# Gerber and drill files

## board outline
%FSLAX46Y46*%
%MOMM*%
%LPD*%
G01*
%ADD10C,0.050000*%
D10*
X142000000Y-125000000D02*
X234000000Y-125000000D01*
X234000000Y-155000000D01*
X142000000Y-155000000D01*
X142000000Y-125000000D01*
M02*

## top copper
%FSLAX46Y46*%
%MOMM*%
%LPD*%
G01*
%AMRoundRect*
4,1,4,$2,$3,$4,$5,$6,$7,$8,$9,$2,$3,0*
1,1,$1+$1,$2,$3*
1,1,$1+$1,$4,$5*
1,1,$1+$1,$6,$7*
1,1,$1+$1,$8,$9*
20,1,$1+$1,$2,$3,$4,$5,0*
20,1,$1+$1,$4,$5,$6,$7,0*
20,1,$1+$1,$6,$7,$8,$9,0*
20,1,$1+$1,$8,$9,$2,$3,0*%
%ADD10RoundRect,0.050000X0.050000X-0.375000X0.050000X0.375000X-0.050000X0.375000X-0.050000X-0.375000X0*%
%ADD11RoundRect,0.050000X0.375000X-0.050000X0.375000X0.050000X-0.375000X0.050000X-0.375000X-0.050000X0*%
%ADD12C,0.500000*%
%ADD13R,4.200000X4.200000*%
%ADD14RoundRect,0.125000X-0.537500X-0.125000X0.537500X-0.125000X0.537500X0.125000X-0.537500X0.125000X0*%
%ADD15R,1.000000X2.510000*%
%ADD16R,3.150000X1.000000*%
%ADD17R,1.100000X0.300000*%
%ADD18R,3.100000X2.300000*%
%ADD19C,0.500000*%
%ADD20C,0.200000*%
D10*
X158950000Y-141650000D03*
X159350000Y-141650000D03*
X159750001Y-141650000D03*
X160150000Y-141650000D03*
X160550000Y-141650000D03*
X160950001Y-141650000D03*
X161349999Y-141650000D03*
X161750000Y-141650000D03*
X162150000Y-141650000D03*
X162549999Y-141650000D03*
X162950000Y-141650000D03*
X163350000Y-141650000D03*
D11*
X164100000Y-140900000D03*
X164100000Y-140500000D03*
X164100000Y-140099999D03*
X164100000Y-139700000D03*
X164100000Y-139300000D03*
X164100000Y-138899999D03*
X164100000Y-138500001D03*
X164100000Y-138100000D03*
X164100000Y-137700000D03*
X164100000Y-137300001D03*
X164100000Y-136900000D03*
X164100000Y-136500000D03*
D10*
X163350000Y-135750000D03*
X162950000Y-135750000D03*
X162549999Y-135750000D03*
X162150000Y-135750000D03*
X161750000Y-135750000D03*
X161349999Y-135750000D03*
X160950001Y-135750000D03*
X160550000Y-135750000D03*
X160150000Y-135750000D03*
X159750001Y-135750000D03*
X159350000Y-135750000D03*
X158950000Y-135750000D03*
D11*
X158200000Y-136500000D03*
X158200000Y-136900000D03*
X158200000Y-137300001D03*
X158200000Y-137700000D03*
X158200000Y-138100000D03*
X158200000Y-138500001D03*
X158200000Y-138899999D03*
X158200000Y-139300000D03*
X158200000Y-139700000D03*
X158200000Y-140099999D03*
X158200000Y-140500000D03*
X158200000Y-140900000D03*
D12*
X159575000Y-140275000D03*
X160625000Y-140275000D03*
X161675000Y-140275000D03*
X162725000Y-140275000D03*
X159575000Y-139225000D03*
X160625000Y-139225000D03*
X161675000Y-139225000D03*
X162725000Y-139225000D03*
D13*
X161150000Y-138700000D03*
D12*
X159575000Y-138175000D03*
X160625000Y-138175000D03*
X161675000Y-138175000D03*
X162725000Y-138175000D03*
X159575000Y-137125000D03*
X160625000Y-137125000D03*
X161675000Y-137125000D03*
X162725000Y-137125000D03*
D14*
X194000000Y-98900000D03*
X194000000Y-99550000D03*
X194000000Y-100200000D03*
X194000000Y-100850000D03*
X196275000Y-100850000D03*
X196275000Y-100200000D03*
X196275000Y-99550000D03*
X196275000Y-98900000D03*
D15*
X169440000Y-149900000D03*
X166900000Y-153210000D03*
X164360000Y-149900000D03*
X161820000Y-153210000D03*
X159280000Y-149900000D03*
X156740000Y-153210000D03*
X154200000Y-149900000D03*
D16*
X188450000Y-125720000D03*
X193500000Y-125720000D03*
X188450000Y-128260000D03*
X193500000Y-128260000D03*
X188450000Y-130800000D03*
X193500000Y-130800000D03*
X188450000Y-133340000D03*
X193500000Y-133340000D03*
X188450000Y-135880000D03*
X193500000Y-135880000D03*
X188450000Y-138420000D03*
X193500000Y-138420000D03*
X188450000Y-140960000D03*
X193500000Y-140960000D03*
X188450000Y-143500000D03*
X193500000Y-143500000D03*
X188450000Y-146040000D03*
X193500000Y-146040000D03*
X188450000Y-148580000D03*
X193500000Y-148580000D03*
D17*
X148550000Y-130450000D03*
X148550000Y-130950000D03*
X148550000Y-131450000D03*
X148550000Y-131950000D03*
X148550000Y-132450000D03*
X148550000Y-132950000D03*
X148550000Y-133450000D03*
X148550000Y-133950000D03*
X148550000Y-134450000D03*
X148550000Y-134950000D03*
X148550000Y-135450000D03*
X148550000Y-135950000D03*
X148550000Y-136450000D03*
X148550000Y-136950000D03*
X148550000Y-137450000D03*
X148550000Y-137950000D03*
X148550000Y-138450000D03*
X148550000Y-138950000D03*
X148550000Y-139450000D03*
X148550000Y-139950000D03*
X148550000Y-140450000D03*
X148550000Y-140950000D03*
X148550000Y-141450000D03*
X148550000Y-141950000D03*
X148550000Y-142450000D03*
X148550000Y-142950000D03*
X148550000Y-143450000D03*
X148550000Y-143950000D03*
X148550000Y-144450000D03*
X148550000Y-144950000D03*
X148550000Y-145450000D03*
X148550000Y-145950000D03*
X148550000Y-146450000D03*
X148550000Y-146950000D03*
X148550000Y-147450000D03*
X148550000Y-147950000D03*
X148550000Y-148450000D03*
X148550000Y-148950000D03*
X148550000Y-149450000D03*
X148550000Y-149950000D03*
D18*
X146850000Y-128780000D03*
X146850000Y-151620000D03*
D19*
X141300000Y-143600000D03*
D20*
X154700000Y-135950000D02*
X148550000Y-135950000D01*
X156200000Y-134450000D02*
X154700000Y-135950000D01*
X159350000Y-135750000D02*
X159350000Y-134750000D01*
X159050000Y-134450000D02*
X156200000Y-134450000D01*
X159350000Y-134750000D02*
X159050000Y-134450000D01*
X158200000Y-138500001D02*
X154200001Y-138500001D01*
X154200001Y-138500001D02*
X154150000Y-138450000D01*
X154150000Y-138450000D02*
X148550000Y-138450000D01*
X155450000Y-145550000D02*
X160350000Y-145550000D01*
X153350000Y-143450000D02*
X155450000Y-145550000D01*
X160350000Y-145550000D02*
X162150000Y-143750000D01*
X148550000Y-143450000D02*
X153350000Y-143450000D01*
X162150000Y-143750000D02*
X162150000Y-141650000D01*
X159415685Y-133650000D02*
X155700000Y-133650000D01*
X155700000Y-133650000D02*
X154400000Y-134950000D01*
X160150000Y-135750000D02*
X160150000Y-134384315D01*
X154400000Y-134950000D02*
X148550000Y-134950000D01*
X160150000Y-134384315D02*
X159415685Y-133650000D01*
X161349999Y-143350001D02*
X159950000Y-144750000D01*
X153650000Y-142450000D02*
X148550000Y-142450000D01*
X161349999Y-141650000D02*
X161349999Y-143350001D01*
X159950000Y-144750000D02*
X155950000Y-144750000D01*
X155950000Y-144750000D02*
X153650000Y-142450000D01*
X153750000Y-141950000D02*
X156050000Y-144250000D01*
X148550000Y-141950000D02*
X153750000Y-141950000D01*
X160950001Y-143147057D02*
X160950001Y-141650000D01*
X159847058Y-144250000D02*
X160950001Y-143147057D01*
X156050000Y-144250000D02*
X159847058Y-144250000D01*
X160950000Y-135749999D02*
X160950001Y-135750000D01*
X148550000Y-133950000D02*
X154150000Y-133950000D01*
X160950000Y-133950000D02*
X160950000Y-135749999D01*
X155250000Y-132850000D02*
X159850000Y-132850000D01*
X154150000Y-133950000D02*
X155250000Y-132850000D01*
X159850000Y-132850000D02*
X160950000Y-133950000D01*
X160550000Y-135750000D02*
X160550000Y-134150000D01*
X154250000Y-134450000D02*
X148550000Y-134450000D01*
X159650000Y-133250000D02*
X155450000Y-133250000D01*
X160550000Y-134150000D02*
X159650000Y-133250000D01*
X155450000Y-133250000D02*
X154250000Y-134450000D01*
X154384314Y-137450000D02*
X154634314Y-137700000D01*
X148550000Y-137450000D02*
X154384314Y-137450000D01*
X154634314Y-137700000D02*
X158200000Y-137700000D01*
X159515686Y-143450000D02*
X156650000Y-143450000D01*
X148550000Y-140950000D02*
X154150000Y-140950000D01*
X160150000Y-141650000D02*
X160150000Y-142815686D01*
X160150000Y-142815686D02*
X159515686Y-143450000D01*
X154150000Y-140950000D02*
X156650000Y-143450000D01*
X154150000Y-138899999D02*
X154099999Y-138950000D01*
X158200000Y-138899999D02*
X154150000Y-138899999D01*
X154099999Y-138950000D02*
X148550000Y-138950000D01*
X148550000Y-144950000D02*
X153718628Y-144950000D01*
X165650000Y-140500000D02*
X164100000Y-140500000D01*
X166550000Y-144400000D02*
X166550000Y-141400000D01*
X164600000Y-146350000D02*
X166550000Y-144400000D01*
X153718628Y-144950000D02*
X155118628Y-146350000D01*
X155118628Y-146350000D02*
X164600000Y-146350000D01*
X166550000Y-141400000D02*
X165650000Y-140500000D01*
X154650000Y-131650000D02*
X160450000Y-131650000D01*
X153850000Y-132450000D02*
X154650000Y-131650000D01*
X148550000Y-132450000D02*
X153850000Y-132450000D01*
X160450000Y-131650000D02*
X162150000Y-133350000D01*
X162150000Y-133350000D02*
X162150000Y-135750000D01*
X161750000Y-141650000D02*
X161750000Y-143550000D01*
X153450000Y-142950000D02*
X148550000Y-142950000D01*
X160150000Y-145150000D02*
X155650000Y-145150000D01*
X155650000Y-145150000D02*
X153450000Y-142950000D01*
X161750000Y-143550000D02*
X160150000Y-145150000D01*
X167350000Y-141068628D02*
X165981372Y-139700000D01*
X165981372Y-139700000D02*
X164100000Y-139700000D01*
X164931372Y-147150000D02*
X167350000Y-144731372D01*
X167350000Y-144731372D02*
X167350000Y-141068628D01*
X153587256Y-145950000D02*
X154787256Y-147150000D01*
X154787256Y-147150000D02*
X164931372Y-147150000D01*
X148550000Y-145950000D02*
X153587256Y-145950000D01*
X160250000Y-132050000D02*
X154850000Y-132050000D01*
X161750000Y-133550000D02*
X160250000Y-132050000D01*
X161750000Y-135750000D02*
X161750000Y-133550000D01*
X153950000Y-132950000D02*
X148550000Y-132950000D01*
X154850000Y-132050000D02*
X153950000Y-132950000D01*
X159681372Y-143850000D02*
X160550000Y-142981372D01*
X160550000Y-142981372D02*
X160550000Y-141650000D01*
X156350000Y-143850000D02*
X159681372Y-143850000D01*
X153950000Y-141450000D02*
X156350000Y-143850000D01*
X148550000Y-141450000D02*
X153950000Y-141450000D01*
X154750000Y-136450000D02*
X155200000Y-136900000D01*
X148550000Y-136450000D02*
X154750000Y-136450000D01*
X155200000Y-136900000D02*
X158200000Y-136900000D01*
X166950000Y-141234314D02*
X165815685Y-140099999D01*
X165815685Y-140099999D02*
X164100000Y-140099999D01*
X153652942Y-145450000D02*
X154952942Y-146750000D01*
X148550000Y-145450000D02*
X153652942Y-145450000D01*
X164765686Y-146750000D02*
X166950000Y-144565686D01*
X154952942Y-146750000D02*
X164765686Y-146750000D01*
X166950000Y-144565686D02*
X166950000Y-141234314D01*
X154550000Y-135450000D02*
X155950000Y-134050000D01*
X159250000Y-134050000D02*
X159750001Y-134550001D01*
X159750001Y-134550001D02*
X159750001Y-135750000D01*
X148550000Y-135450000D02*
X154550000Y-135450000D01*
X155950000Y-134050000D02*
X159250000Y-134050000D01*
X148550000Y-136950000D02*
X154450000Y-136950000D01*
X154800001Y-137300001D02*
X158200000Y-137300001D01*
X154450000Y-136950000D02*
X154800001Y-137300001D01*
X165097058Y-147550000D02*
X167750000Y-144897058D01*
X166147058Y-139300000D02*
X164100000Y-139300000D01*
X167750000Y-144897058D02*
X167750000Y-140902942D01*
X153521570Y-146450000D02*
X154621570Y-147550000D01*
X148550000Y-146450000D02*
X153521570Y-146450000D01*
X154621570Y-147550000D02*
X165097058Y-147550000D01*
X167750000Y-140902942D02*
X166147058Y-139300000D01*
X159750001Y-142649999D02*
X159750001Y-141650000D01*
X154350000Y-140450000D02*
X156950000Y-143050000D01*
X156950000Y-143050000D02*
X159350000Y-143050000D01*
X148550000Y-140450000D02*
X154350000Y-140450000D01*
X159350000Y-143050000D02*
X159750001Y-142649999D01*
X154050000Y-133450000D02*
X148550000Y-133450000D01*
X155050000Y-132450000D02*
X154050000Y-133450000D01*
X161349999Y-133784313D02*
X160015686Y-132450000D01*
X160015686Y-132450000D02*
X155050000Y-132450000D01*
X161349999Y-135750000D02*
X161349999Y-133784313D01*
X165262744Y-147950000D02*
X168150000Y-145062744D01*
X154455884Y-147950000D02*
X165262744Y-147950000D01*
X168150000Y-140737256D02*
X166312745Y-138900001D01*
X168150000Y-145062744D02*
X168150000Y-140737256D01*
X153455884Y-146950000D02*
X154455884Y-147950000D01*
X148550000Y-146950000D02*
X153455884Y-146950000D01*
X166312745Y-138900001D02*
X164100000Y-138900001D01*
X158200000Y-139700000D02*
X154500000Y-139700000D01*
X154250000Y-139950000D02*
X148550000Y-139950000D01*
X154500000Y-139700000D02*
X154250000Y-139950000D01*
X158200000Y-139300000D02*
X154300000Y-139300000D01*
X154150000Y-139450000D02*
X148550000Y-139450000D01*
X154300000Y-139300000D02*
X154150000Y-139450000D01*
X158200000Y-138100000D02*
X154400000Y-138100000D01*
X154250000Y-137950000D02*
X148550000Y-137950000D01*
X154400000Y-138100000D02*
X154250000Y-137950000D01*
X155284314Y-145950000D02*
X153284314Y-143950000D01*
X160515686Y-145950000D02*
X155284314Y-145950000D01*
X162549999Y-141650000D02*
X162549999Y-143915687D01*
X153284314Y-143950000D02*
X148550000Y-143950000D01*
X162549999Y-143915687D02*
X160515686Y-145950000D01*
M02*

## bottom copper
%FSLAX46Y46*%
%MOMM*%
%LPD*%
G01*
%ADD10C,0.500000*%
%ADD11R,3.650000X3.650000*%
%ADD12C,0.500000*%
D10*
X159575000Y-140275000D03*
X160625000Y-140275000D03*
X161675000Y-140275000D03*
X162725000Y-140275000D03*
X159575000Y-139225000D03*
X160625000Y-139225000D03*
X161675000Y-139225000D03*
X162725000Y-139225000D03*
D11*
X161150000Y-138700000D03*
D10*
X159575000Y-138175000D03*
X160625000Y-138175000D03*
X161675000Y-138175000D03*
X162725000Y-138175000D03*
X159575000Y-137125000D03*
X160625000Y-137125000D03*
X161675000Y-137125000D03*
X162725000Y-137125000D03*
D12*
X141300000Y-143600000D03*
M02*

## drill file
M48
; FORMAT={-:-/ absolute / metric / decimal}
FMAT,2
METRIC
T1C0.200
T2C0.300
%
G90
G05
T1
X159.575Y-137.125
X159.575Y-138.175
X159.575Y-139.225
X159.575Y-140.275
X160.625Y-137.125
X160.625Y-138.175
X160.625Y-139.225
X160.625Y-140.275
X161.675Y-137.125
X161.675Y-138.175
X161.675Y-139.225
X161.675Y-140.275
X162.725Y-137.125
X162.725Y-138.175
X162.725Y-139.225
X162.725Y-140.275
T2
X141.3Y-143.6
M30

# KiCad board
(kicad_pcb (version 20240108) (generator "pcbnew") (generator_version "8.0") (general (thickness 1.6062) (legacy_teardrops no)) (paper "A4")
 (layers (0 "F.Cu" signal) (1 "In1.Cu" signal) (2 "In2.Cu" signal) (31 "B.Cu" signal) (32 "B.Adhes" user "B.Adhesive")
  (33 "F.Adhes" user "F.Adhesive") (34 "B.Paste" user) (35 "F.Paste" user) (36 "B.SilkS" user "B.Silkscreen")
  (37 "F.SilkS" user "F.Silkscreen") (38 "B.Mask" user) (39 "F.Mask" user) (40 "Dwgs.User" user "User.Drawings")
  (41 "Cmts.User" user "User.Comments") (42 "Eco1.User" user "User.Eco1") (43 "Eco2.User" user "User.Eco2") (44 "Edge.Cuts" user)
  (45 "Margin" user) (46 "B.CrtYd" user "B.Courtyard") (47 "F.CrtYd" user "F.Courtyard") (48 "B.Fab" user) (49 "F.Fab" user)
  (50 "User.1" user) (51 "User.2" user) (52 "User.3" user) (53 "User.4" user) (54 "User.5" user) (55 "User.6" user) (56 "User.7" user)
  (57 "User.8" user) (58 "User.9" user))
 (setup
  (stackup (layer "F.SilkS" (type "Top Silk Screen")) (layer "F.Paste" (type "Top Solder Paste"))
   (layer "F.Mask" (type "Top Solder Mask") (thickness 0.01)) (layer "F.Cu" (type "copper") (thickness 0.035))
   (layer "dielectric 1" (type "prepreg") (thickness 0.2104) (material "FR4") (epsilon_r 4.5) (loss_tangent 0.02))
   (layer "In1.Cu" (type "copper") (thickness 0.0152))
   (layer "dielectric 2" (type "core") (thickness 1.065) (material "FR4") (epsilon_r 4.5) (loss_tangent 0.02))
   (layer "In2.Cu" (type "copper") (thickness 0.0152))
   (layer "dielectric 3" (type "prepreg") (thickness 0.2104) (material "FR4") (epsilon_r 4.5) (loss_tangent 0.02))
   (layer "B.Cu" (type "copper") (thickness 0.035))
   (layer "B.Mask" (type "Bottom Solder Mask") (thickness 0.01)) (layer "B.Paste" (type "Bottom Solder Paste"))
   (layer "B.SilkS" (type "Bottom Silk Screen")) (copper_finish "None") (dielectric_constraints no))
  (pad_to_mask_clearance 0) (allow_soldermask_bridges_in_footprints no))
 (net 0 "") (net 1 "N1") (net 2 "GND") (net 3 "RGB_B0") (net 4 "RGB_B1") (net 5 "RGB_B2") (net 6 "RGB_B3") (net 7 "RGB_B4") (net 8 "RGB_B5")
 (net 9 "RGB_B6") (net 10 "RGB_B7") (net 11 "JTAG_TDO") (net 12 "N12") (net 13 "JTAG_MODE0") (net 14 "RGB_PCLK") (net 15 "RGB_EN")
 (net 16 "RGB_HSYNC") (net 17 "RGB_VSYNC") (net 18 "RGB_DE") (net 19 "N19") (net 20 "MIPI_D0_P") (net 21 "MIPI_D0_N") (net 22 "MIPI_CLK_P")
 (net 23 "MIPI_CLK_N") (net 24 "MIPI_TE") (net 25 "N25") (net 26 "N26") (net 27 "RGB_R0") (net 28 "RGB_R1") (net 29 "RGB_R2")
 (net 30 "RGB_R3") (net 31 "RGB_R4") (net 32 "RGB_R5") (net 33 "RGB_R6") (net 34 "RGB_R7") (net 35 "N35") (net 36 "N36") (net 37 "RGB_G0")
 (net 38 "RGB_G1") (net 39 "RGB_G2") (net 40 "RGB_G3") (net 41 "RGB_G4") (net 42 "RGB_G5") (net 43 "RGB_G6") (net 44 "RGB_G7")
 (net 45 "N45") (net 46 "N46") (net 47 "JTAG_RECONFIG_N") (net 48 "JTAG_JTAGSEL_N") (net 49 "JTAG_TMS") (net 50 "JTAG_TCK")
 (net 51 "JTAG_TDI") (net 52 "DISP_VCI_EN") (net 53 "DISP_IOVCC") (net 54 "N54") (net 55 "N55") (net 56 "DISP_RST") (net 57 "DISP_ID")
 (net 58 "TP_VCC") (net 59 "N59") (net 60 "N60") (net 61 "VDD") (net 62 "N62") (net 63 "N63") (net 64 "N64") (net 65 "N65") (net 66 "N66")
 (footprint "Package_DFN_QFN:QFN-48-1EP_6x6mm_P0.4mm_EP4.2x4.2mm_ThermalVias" (layer "F.Cu") (at 161.15 138.7 90)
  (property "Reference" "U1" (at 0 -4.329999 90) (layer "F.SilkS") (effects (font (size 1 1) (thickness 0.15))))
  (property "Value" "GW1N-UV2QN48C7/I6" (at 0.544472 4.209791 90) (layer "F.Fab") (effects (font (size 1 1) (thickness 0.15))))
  (pad "" smd custom (at -1.8375 -1.8375 90) (size 0.295204 0.295204) (layers "F.Paste") (options (clearance outline) (anchor circle))
   (primitives))
  (pad "" smd custom (at -1.8375 -1.05 90) (size 0.331171 0.331171) (layers "F.Paste") (options (clearance outline) (anchor circle))
   (primitives))
  (pad "" smd custom (at -1.8375 0 90) (size 0.331171 0.331171) (layers "F.Paste") (options (clearance outline) (anchor circle))
   (primitives))
  (pad "" smd custom (at -1.8375 1.05 90) (size 0.331171 0.331171) (layers "F.Paste") (options (clearance outline) (anchor circle))
   (primitives))
  (pad "" smd custom (at -1.8375 1.8375 90) (size 0.295204 0.295204) (layers "F.Paste") (options (clearance outline) (anchor circle))
   (primitives))
  (pad "" smd custom (at -1.05 -1.8375 90) (size 0.331171 0.331171) (layers "F.Paste") (options (clearance outline) (anchor circle))
   (primitives))
  (pad "" smd roundrect (at -1.05 -1.05 90) (size 0.846537 0.846537) (layers "F.Paste") (roundrect_rratio 0.25))
  (pad "" smd roundrect (at -1.05 0 90) (size 0.846537 0.846537) (layers "F.Paste") (roundrect_rratio 0.25))
  (pad "" smd roundrect (at -1.05 1.05 90) (size 0.846537 0.846537) (layers "F.Paste") (roundrect_rratio 0.25))
  (pad "" smd custom (at -1.05 1.8375 90) (size 0.331171 0.331171) (layers "F.Paste") (options (clearance outline) (anchor circle))
   (primitives))
  (pad "" smd custom (at 0 -1.8375 90) (size 0.331171 0.331171) (layers "F.Paste") (options (clearance outline) (anchor circle))
   (primitives))
  (pad "" smd roundrect (at 0 -1.05 90) (size 0.846537 0.846537) (layers "F.Paste") (roundrect_rratio 0.25))
  (pad "" smd roundrect (at 0 0 90) (size 0.846537 0.846537) (layers "F.Paste") (roundrect_rratio 0.25))
  (pad "" smd roundrect (at 0 1.05 90) (size 0.846537 0.846537) (layers "F.Paste") (roundrect_rratio 0.25))
  (pad "" smd custom (at 0 1.8375 90) (size 0.331171 0.331171) (layers "F.Paste") (options (clearance outline) (anchor circle)) (primitives))
  (pad "" smd custom (at 1.05 -1.8375 90) (size 0.331171 0.331171) (layers "F.Paste") (options (clearance outline) (anchor circle))
   (primitives))
  (pad "" smd roundrect (at 1.05 -1.05 90) (size 0.846537 0.846537) (layers "F.Paste") (roundrect_rratio 0.25))
  (pad "" smd roundrect (at 1.05 0 90) (size 0.846537 0.846537) (layers "F.Paste") (roundrect_rratio 0.25))
  (pad "" smd roundrect (at 1.05 1.05 90) (size 0.846537 0.846537) (layers "F.Paste") (roundrect_rratio 0.25))
  (pad "" smd custom (at 1.05 1.8375 90) (size 0.331171 0.331171) (layers "F.Paste") (options (clearance outline) (anchor circle))
   (primitives))
  (pad "" smd custom (at 1.8375 -1.8375 90) (size 0.295204 0.295204) (layers "F.Paste") (options (clearance outline) (anchor circle))
   (primitives))
  (pad "" smd custom (at 1.8375 -1.05 90) (size 0.331171 0.331171) (layers "F.Paste") (options (clearance outline) (anchor circle))
   (primitives))
  (pad "" smd custom (at 1.8375 0 90) (size 0.331171 0.331171) (layers "F.Paste") (options (clearance outline) (anchor circle)) (primitives))
  (pad "" smd custom (at 1.8375 1.05 90) (size 0.331171 0.331171) (layers "F.Paste") (options (clearance outline) (anchor circle))
   (primitives))
  (pad "" smd custom (at 1.8375 1.8375 90) (size 0.295204 0.295204) (layers "F.Paste") (options (clearance outline) (anchor circle))
   (primitives))
  (pad "1" smd roundrect (at -2.95 -2.2 90) (size 0.85 0.2) (layers "F.Cu" "F.Paste" "F.Mask") (roundrect_rratio 0.25) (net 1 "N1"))
  (pad "2" smd roundrect (at -2.95 -1.8 90) (size 0.85 0.2) (layers "F.Cu" "F.Paste" "F.Mask") (roundrect_rratio 0.25) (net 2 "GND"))
  (pad "3" smd roundrect (at -2.95 -1.399999 90) (size 0.85 0.2) (layers "F.Cu" "F.Paste" "F.Mask") (roundrect_rratio 0.25) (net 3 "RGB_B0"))
  (pad "4" smd roundrect (at -2.95 -1 90) (size 0.85 0.2) (layers "F.Cu" "F.Paste" "F.Mask") (roundrect_rratio 0.25) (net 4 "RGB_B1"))
  (pad "5" smd roundrect (at -2.95 -0.6 90) (size 0.85 0.2) (layers "F.Cu" "F.Paste" "F.Mask") (roundrect_rratio 0.25) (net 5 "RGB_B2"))
  (pad "6" smd roundrect (at -2.95 -0.199999 90) (size 0.85 0.2) (layers "F.Cu" "F.Paste" "F.Mask") (roundrect_rratio 0.25) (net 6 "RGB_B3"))
  (pad "7" smd roundrect (at -2.95 0.199999 90) (size 0.85 0.2) (layers "F.Cu" "F.Paste" "F.Mask") (roundrect_rratio 0.25) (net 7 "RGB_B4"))
  (pad "8" smd roundrect (at -2.95 0.6 90) (size 0.85 0.2) (layers "F.Cu" "F.Paste" "F.Mask") (roundrect_rratio 0.25) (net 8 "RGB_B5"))
  (pad "9" smd roundrect (at -2.95 1 90) (size 0.85 0.2) (layers "F.Cu" "F.Paste" "F.Mask") (roundrect_rratio 0.25) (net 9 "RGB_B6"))
  (pad "10" smd roundrect (at -2.95 1.399999 90) (size 0.85 0.2) (layers "F.Cu" "F.Paste" "F.Mask") (roundrect_rratio 0.25)
   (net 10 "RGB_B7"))
  (pad "11" smd roundrect (at -2.95 1.8 90) (size 0.85 0.2) (layers "F.Cu" "F.Paste" "F.Mask") (roundrect_rratio 0.25) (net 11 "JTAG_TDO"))
  (pad "12" smd roundrect (at -2.95 2.2 90) (size 0.85 0.2) (layers "F.Cu" "F.Paste" "F.Mask") (roundrect_rratio 0.25) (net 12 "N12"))
  (pad "13" smd roundrect (at -2.2 2.95 90) (size 0.2 0.85) (layers "F.Cu" "F.Paste" "F.Mask") (roundrect_rratio 0.25) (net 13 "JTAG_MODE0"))
  (pad "14" smd roundrect (at -1.8 2.95 90) (size 0.2 0.85) (layers "F.Cu" "F.Paste" "F.Mask") (roundrect_rratio 0.25) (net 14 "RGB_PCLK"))
  (pad "15" smd roundrect (at -1.399999 2.95 90) (size 0.2 0.85) (layers "F.Cu" "F.Paste" "F.Mask") (roundrect_rratio 0.25)
   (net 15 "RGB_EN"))
  (pad "16" smd roundrect (at -1 2.95 90) (size 0.2 0.85) (layers "F.Cu" "F.Paste" "F.Mask") (roundrect_rratio 0.25) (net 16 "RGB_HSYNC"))
  (pad "17" smd roundrect (at -0.6 2.95 90) (size 0.2 0.85) (layers "F.Cu" "F.Paste" "F.Mask") (roundrect_rratio 0.25) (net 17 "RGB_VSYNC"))
  (pad "18" smd roundrect (at -0.199999 2.95 90) (size 0.2 0.85) (layers "F.Cu" "F.Paste" "F.Mask") (roundrect_rratio 0.25)
   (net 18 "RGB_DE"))
  (pad "19" smd roundrect (at 0.199999 2.95 90) (size 0.2 0.85) (layers "F.Cu" "F.Paste" "F.Mask") (roundrect_rratio 0.25) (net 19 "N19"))
  (pad "20" smd roundrect (at 0.6 2.95 90) (size 0.2 0.85) (layers "F.Cu" "F.Paste" "F.Mask") (roundrect_rratio 0.25) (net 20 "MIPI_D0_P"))
  (pad "21" smd roundrect (at 1 2.95 90) (size 0.2 0.85) (layers "F.Cu" "F.Paste" "F.Mask") (roundrect_rratio 0.25) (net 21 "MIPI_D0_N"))
  (pad "22" smd roundrect (at 1.399999 2.95 90) (size 0.2 0.85) (layers "F.Cu" "F.Paste" "F.Mask") (roundrect_rratio 0.25)
   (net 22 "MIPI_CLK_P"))
  (pad "23" smd roundrect (at 1.8 2.95 90) (size 0.2 0.85) (layers "F.Cu" "F.Paste" "F.Mask") (roundrect_rratio 0.25) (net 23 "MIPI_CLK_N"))
  (pad "24" smd roundrect (at 2.2 2.95 90) (size 0.2 0.85) (layers "F.Cu" "F.Paste" "F.Mask") (roundrect_rratio 0.25) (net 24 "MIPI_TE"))
  (pad "25" smd roundrect (at 2.95 2.2 90) (size 0.85 0.2) (layers "F.Cu" "F.Paste" "F.Mask") (roundrect_rratio 0.25) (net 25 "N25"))
  (pad "26" smd roundrect (at 2.95 1.8 90) (size 0.85 0.2) (layers "F.Cu" "F.Paste" "F.Mask") (roundrect_rratio 0.25) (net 2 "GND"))
  (pad "27" smd roundrect (at 2.95 1.399999 90) (size 0.85 0.2) (layers "F.Cu" "F.Paste" "F.Mask") (roundrect_rratio 0.25) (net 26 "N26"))
  (pad "28" smd roundrect (at 2.95 1 90) (size 0.85 0.2) (layers "F.Cu" "F.Paste" "F.Mask") (roundrect_rratio 0.25) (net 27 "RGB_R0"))
  (pad "29" smd roundrect (at 2.95 0.6 90) (size 0.85 0.2) (layers "F.Cu" "F.Paste" "F.Mask") (roundrect_rratio 0.25) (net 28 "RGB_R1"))
  (pad "30" smd roundrect (at 2.95 0.199999 90) (size 0.85 0.2) (layers "F.Cu" "F.Paste" "F.Mask") (roundrect_rratio 0.25) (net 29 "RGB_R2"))
  (pad "31" smd roundrect (at 2.95 -0.199999 90) (size 0.85 0.2) (layers "F.Cu" "F.Paste" "F.Mask") (roundrect_rratio 0.25)
   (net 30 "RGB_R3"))
  (pad "32" smd roundrect (at 2.95 -0.6 90) (size 0.85 0.2) (layers "F.Cu" "F.Paste" "F.Mask") (roundrect_rratio 0.25) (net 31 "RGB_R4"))
  (pad "33" smd roundrect (at 2.95 -1 90) (size 0.85 0.2) (layers "F.Cu" "F.Paste" "F.Mask") (roundrect_rratio 0.25) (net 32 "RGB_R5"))
  (pad "34" smd roundrect (at 2.95 -1.399999 90) (size 0.85 0.2) (layers "F.Cu" "F.Paste" "F.Mask") (roundrect_rratio 0.25)
   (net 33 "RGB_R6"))
  (pad "35" smd roundrect (at 2.95 -1.8 90) (size 0.85 0.2) (layers "F.Cu" "F.Paste" "F.Mask") (roundrect_rratio 0.25) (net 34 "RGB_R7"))
  (pad "36" smd roundrect (at 2.95 -2.2 90) (size 0.85 0.2) (layers "F.Cu" "F.Paste" "F.Mask") (roundrect_rratio 0.25) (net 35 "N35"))
  (pad "37" smd roundrect (at 2.2 -2.95 90) (size 0.2 0.85) (layers "F.Cu" "F.Paste" "F.Mask") (roundrect_rratio 0.25) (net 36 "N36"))
  (pad "38" smd roundrect (at 1.8 -2.95 90) (size 0.2 0.85) (layers "F.Cu" "F.Paste" "F.Mask") (roundrect_rratio 0.25) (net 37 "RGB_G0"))
  (pad "39" smd roundrect (at 1.399999 -2.95 90) (size 0.2 0.85) (layers "F.Cu" "F.Paste" "F.Mask") (roundrect_rratio 0.25)
   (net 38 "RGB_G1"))
  (pad "40" smd roundrect (at 1 -2.95 90) (size 0.2 0.85) (layers "F.Cu" "F.Paste" "F.Mask") (roundrect_rratio 0.25) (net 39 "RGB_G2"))
  (pad "41" smd roundrect (at 0.6 -2.95 90) (size 0.2 0.85) (layers "F.Cu" "F.Paste" "F.Mask") (roundrect_rratio 0.25) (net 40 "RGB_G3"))
  (pad "42" smd roundrect (at 0.199999 -2.95 90) (size 0.2 0.85) (layers "F.Cu" "F.Paste" "F.Mask") (roundrect_rratio 0.25)
   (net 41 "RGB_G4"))
  (pad "43" smd roundrect (at -0.199999 -2.95 90) (size 0.2 0.85) (layers "F.Cu" "F.Paste" "F.Mask") (roundrect_rratio 0.25)
   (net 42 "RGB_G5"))
  (pad "44" smd roundrect (at -0.6 -2.95 90) (size 0.2 0.85) (layers "F.Cu" "F.Paste" "F.Mask") (roundrect_rratio 0.25) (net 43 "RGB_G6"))
  (pad "45" smd roundrect (at -1 -2.95 90) (size 0.2 0.85) (layers "F.Cu" "F.Paste" "F.Mask") (roundrect_rratio 0.25) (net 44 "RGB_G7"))
  (pad "46" smd roundrect (at -1.399999 -2.95 90) (size 0.2 0.85) (layers "F.Cu" "F.Paste" "F.Mask") (roundrect_rratio 0.25) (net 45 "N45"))
  (pad "47" smd roundrect (at -1.8 -2.95 90) (size 0.2 0.85) (layers "F.Cu" "F.Paste" "F.Mask") (roundrect_rratio 0.25) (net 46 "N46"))
  (pad "48" smd roundrect (at -2.2 -2.95 90) (size 0.2 0.85) (layers "F.Cu" "F.Paste" "F.Mask") (roundrect_rratio 0.25)
   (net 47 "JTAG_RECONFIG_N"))
  (pad "49" thru_hole circle (at -1.575 -1.575 90) (size 0.5 0.5) (drill 0.2) (layers "*.Cu") (remove_unused_layers no))
  (pad "49" thru_hole circle (at -1.575 -0.525 90) (size 0.5 0.5) (drill 0.2) (layers "*.Cu") (remove_unused_layers no))
  (pad "49" thru_hole circle (at -1.575 0.525 90) (size 0.5 0.5) (drill 0.2) (layers "*.Cu") (remove_unused_layers no))
  (pad "49" thru_hole circle (at -1.575 1.575 90) (size 0.5 0.5) (drill 0.2) (layers "*.Cu") (remove_unused_layers no))
  (pad "49" thru_hole circle (at -0.525 -1.575 90) (size 0.5 0.5) (drill 0.2) (layers "*.Cu") (remove_unused_layers no))
  (pad "49" thru_hole circle (at -0.525 -0.525 90) (size 0.5 0.5) (drill 0.2) (layers "*.Cu") (remove_unused_layers no))
  (pad "49" thru_hole circle (at -0.525 0.525 90) (size 0.5 0.5) (drill 0.2) (layers "*.Cu") (remove_unused_layers no))
  (pad "49" thru_hole circle (at -0.525 1.575 90) (size 0.5 0.5) (drill 0.2) (layers "*.Cu") (remove_unused_layers no))
  (pad "49" smd rect (at 0 0 90) (size 3.65 3.65) (layers "B.Cu") (zone_connect 2))
  (pad "49" smd rect (at 0 0 90) (size 4.2 4.2) (layers "F.Cu" "F.Mask") (zone_connect 2))
  (pad "49" thru_hole circle (at 0.525 -1.575 90) (size 0.5 0.5) (drill 0.2) (layers "*.Cu") (remove_unused_layers no))
  (pad "49" thru_hole circle (at 0.525 -0.525 90) (size 0.5 0.5) (drill 0.2) (layers "*.Cu") (remove_unused_layers no))
  (pad "49" thru_hole circle (at 0.525 0.525 90) (size 0.5 0.5) (drill 0.2) (layers "*.Cu") (remove_unused_layers no))
  (pad "49" thru_hole circle (at 0.525 1.575 90) (size 0.5 0.5) (drill 0.2) (layers "*.Cu") (remove_unused_layers no))
  (pad "49" thru_hole circle (at 1.575 -1.575 90) (size 0.5 0.5) (drill 0.2) (layers "*.Cu") (remove_unused_layers no))
  (pad "49" thru_hole circle (at 1.575 -0.525 90) (size 0.5 0.5) (drill 0.2) (layers "*.Cu") (remove_unused_layers no))
  (pad "49" thru_hole circle (at 1.575 0.525 90) (size 0.5 0.5) (drill 0.2) (layers "*.Cu") (remove_unused_layers no))
  (pad "49" thru_hole circle (at 1.575 1.575 90) (size 0.5 0.5) (drill 0.2) (layers "*.Cu") (remove_unused_layers no)))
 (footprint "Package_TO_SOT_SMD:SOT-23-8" (layer "F.Cu") (at 195.1375 99.875)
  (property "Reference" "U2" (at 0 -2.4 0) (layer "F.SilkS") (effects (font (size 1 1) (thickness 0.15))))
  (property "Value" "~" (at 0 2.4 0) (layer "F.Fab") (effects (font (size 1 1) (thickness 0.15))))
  (pad "1" smd roundrect (at -1.1375 -0.975) (size 1.325 0.5) (layers "F.Cu" "F.Paste" "F.Mask") (roundrect_rratio 0.25))
  (pad "2" smd roundrect (at -1.1375 -0.325) (size 1.325 0.5) (layers "F.Cu" "F.Paste" "F.Mask") (roundrect_rratio 0.25))
  (pad "3" smd roundrect (at -1.1375 0.325) (size 1.325 0.5) (layers "F.Cu" "F.Paste" "F.Mask") (roundrect_rratio 0.25))
  (pad "4" smd roundrect (at -1.1375 0.975) (size 1.325 0.5) (layers "F.Cu" "F.Paste" "F.Mask") (roundrect_rratio 0.25))
  (pad "5" smd roundrect (at 1.1375 0.975) (size 1.325 0.5) (layers "F.Cu" "F.Paste" "F.Mask") (roundrect_rratio 0.25))
  (pad "6" smd roundrect (at 1.1375 0.325) (size 1.325 0.5) (layers "F.Cu" "F.Paste" "F.Mask") (roundrect_rratio 0.25))
  (pad "7" smd roundrect (at 1.1375 -0.325) (size 1.325 0.5) (layers "F.Cu" "F.Paste" "F.Mask") (roundrect_rratio 0.25))
  (pad "8" smd roundrect (at 1.1375 -0.975) (size 1.325 0.5) (layers "F.Cu" "F.Paste" "F.Mask") (roundrect_rratio 0.25)))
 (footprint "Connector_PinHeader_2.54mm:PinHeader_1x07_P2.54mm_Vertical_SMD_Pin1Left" (layer "F.Cu") (at 161.82 151.555 -90)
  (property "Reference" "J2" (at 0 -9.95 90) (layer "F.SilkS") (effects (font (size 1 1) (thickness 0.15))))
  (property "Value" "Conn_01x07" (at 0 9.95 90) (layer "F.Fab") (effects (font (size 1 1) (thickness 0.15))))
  (pad "1" smd rect (at -1.655 -7.62 270) (size 2.51 1) (layers "F.Cu" "F.Paste" "F.Mask") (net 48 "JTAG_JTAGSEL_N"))
  (pad "2" smd rect (at 1.655 -5.08 270) (size 2.51 1) (layers "F.Cu" "F.Paste" "F.Mask") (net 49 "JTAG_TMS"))
  (pad "3" smd rect (at -1.655 -2.54 270) (size 2.51 1) (layers "F.Cu" "F.Paste" "F.Mask") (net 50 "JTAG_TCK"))
  (pad "4" smd rect (at 1.655 0 270) (size 2.51 1) (layers "F.Cu" "F.Paste" "F.Mask") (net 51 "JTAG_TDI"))
  (pad "5" smd rect (at -1.655 2.54 270) (size 2.51 1) (layers "F.Cu" "F.Paste" "F.Mask") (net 11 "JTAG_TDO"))
  (pad "6" smd rect (at 1.655 5.08 270) (size 2.51 1) (layers "F.Cu" "F.Paste" "F.Mask") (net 13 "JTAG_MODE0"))
  (pad "7" smd rect (at -1.655 7.62 270) (size 2.51 1) (layers "F.Cu" "F.Paste" "F.Mask") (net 47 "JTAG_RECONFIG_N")))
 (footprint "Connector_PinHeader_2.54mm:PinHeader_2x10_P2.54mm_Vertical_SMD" (layer "F.Cu") (at 190.975 137.15)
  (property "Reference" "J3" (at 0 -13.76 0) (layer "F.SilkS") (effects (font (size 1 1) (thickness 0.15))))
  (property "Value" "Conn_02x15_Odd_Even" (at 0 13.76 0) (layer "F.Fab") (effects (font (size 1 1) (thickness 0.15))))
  (pad "1" smd rect (at -2.525 -11.43) (size 3.15 1) (layers "F.Cu" "F.Paste" "F.Mask") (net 2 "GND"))
  (pad "2" smd rect (at 2.525 -11.43) (size 3.15 1) (layers "F.Cu" "F.Paste" "F.Mask") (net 2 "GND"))
  (pad "3" smd rect (at -2.525 -8.89) (size 3.15 1) (layers "F.Cu" "F.Paste" "F.Mask") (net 23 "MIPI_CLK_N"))
  (pad "4" smd rect (at 2.525 -8.89) (size 3.15 1) (layers "F.Cu" "F.Paste" "F.Mask") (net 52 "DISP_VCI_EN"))
  (pad "5" smd rect (at -2.525 -6.35) (size 3.15 1) (layers "F.Cu" "F.Paste" "F.Mask") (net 22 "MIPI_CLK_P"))
  (pad "6" smd rect (at 2.525 -6.35) (size 3.15 1) (layers "F.Cu" "F.Paste" "F.Mask") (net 2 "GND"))
  (pad "7" smd rect (at -2.525 -3.81) (size 3.15 1) (layers "F.Cu" "F.Paste" "F.Mask") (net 2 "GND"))
  (pad "8" smd rect (at 2.525 -3.81) (size 3.15 1) (layers "F.Cu" "F.Paste" "F.Mask") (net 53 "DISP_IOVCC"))
  (pad "9" smd rect (at -2.525 -1.27) (size 3.15 1) (layers "F.Cu" "F.Paste" "F.Mask") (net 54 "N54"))
  (pad "10" smd rect (at 2.525 -1.27) (size 3.15 1) (layers "F.Cu" "F.Paste" "F.Mask") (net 2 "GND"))
  (pad "11" smd rect (at -2.525 1.27) (size 3.15 1) (layers "F.Cu" "F.Paste" "F.Mask") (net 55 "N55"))
  (pad "12" smd rect (at 2.525 1.27) (size 3.15 1) (layers "F.Cu" "F.Paste" "F.Mask") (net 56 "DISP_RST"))
  (pad "13" smd rect (at -2.525 3.81) (size 3.15 1) (layers "F.Cu" "F.Paste" "F.Mask") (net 2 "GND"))
  (pad "14" smd rect (at 2.525 3.81) (size 3.15 1) (layers "F.Cu" "F.Paste" "F.Mask") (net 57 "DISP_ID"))
  (pad "15" smd rect (at -2.525 6.35) (size 3.15 1) (layers "F.Cu" "F.Paste" "F.Mask") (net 21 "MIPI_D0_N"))
  (pad "16" smd rect (at 2.525 6.35) (size 3.15 1) (layers "F.Cu" "F.Paste" "F.Mask") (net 2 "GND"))
  (pad "17" smd rect (at -2.525 8.89) (size 3.15 1) (layers "F.Cu" "F.Paste" "F.Mask") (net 20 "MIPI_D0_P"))
  (pad "18" smd rect (at 2.525 8.89) (size 3.15 1) (layers "F.Cu" "F.Paste" "F.Mask") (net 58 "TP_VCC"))
  (pad "19" smd rect (at -2.525 11.43) (size 3.15 1) (layers "F.Cu" "F.Paste" "F.Mask") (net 2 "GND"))
  (pad "20" smd rect (at 2.525 11.43) (size 3.15 1) (layers "F.Cu" "F.Paste" "F.Mask") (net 2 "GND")))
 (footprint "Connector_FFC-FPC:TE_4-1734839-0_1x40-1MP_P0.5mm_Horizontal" (layer "F.Cu") (at 147.2 140.2 -90)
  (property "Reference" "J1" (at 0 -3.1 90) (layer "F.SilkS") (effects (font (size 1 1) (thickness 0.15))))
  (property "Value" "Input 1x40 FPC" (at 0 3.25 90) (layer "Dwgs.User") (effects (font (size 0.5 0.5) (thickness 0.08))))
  (pad "1" smd rect (at -9.75 -1.35 270) (size 0.3 1.1) (layers "F.Cu" "F.Paste" "F.Mask") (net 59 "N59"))
  (pad "2" smd rect (at -9.25 -1.35 270) (size 0.3 1.1) (layers "F.Cu" "F.Paste" "F.Mask") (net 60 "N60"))
  (pad "3" smd rect (at -8.75 -1.35 270) (size 0.3 1.1) (layers "F.Cu" "F.Paste" "F.Mask") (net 2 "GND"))
  (pad "4" smd rect (at -8.25 -1.35 270) (size 0.3 1.1) (layers "F.Cu" "F.Paste" "F.Mask") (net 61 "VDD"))
  (pad "5" smd rect (at -7.75 -1.35 270) (size 0.3 1.1) (layers "F.Cu" "F.Paste" "F.Mask") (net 27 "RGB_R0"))
  (pad "6" smd rect (at -7.25 -1.35 270) (size 0.3 1.1) (layers "F.Cu" "F.Paste" "F.Mask") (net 28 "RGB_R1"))
  (pad "7" smd rect (at -6.75 -1.35 270) (size 0.3 1.1) (layers "F.Cu" "F.Paste" "F.Mask") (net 29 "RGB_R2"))
  (pad "8" smd rect (at -6.25 -1.35 270) (size 0.3 1.1) (layers "F.Cu" "F.Paste" "F.Mask") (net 30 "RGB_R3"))
  (pad "9" smd rect (at -5.75 -1.35 270) (size 0.3 1.1) (layers "F.Cu" "F.Paste" "F.Mask") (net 31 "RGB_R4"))
  (pad "10" smd rect (at -5.25 -1.35 270) (size 0.3 1.1) (layers "F.Cu" "F.Paste" "F.Mask") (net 32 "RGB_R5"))
  (pad "11" smd rect (at -4.75 -1.35 270) (size 0.3 1.1) (layers "F.Cu" "F.Paste" "F.Mask") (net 33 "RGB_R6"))
  (pad "12" smd rect (at -4.25 -1.35 270) (size 0.3 1.1) (layers "F.Cu" "F.Paste" "F.Mask") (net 34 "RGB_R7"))
  (pad "13" smd rect (at -3.75 -1.35 270) (size 0.3 1.1) (layers "F.Cu" "F.Paste" "F.Mask") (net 37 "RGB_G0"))
  (pad "14" smd rect (at -3.25 -1.35 270) (size 0.3 1.1) (layers "F.Cu" "F.Paste" "F.Mask") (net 38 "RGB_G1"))
  (pad "15" smd rect (at -2.75 -1.35 270) (size 0.3 1.1) (layers "F.Cu" "F.Paste" "F.Mask") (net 39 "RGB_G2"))
  (pad "16" smd rect (at -2.25 -1.35 270) (size 0.3 1.1) (layers "F.Cu" "F.Paste" "F.Mask") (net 40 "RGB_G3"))
  (pad "17" smd rect (at -1.75 -1.35 270) (size 0.3 1.1) (layers "F.Cu" "F.Paste" "F.Mask") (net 41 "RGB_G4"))
  (pad "18" smd rect (at -1.25 -1.35 270) (size 0.3 1.1) (layers "F.Cu" "F.Paste" "F.Mask") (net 42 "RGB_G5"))
  (pad "19" smd rect (at -0.75 -1.35 270) (size 0.3 1.1) (layers "F.Cu" "F.Paste" "F.Mask") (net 43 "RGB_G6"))
  (pad "20" smd rect (at -0.25 -1.35 270) (size 0.3 1.1) (layers "F.Cu" "F.Paste" "F.Mask") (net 44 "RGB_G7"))
  (pad "21" smd rect (at 0.25 -1.35 270) (size 0.3 1.1) (layers "F.Cu" "F.Paste" "F.Mask") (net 3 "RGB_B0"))
  (pad "22" smd rect (at 0.75 -1.35 270) (size 0.3 1.1) (layers "F.Cu" "F.Paste" "F.Mask") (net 4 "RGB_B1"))
  (pad "23" smd rect (at 1.25 -1.35 270) (size 0.3 1.1) (layers "F.Cu" "F.Paste" "F.Mask") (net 5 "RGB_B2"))
  (pad "24" smd rect (at 1.75 -1.35 270) (size 0.3 1.1) (layers "F.Cu" "F.Paste" "F.Mask") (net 6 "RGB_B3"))
  (pad "25" smd rect (at 2.25 -1.35 270) (size 0.3 1.1) (layers "F.Cu" "F.Paste" "F.Mask") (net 7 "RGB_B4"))
  (pad "26" smd rect (at 2.75 -1.35 270) (size 0.3 1.1) (layers "F.Cu" "F.Paste" "F.Mask") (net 8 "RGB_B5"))
  (pad "27" smd rect (at 3.25 -1.35 270) (size 0.3 1.1) (layers "F.Cu" "F.Paste" "F.Mask") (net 9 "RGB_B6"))
  (pad "28" smd rect (at 3.75 -1.35 270) (size 0.3 1.1) (layers "F.Cu" "F.Paste" "F.Mask") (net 10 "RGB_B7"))
  (pad "29" smd rect (at 4.25 -1.35 270) (size 0.3 1.1) (layers "F.Cu" "F.Paste" "F.Mask") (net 2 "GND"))
  (pad "30" smd rect (at 4.75 -1.35 270) (size 0.3 1.1) (layers "F.Cu" "F.Paste" "F.Mask") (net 14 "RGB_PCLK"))
  (pad "31" smd rect (at 5.25 -1.35 270) (size 0.3 1.1) (layers "F.Cu" "F.Paste" "F.Mask") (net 15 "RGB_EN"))
  (pad "32" smd rect (at 5.75 -1.35 270) (size 0.3 1.1) (layers "F.Cu" "F.Paste" "F.Mask") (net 16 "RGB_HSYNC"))
  (pad "33" smd rect (at 6.25 -1.35 270) (size 0.3 1.1) (layers "F.Cu" "F.Paste" "F.Mask") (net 17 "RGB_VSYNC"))
  (pad "34" smd rect (at 6.75 -1.35 270) (size 0.3 1.1) (layers "F.Cu" "F.Paste" "F.Mask") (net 18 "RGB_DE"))
  (pad "35" smd rect (at 7.25 -1.35 270) (size 0.3 1.1) (layers "F.Cu" "F.Paste" "F.Mask") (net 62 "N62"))
  (pad "36" smd rect (at 7.75 -1.35 270) (size 0.3 1.1) (layers "F.Cu" "F.Paste" "F.Mask") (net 2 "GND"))
  (pad "37" smd rect (at 8.25 -1.35 270) (size 0.3 1.1) (layers "F.Cu" "F.Paste" "F.Mask") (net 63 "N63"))
  (pad "38" smd rect (at 8.75 -1.35 270) (size 0.3 1.1) (layers "F.Cu" "F.Paste" "F.Mask") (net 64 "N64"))
  (pad "39" smd rect (at 9.25 -1.35 270) (size 0.3 1.1) (layers "F.Cu" "F.Paste" "F.Mask") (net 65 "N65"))
  (pad "40" smd rect (at 9.75 -1.35 270) (size 0.3 1.1) (layers "F.Cu" "F.Paste" "F.Mask") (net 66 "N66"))
  (pad "MP" smd rect (at -11.42 0.35 270) (size 2.3 3.1) (layers "F.Cu" "F.Paste" "F.Mask"))
  (pad "MP" smd rect (at 11.42 0.35 270) (size 2.3 3.1) (layers "F.Cu" "F.Paste" "F.Mask")))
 (gr_rect (start 142 125) (end 234 155) (stroke (width 0.05) (type default)) (fill none) (layer "Edge.Cuts"))
 (via (at 141.3 143.6) (size 0.5) (drill 0.3) (layers "F.Cu" "B.Cu") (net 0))
 (segment (start 154.7 135.95) (end 148.55 135.95) (width 0.2) (layer "F.Cu") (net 34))
 (segment (start 156.2 134.45) (end 154.7 135.95) (width 0.2) (layer "F.Cu") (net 34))
 (segment (start 159.35 135.75) (end 159.35 134.75) (width 0.2) (layer "F.Cu") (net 34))
 (segment (start 159.05 134.45) (end 156.2 134.45) (width 0.2) (layer "F.Cu") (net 34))
 (segment (start 159.35 134.75) (end 159.05 134.45) (width 0.2) (layer "F.Cu") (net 34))
 (segment (start 158.2 138.500001) (end 154.200001 138.500001) (width 0.2) (layer "F.Cu") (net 41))
 (segment (start 154.200001 138.500001) (end 154.15 138.45) (width 0.2) (layer "F.Cu") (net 41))
 (segment (start 154.15 138.45) (end 148.55 138.45) (width 0.2) (layer "F.Cu") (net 41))
 (segment (start 155.45 145.55) (end 160.35 145.55) (width 0.2) (layer "F.Cu") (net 9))
 (segment (start 153.35 143.45) (end 155.45 145.55) (width 0.2) (layer "F.Cu") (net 9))
 (segment (start 160.35 145.55) (end 162.15 143.75) (width 0.2) (layer "F.Cu") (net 9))
 (segment (start 148.55 143.45) (end 153.35 143.45) (width 0.2) (layer "F.Cu") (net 9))
 (segment (start 162.15 143.75) (end 162.15 141.65) (width 0.2) (layer "F.Cu") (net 9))
 (segment (start 159.415685 133.65) (end 155.7 133.65) (width 0.2) (layer "F.Cu") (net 32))
 (segment (start 155.7 133.65) (end 154.4 134.95) (width 0.2) (layer "F.Cu") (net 32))
 (segment (start 160.15 135.75) (end 160.15 134.384315) (width 0.2) (layer "F.Cu") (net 32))
 (segment (start 154.4 134.95) (end 148.55 134.95) (width 0.2) (layer "F.Cu") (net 32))
 (segment (start 160.15 134.384315) (end 159.415685 133.65) (width 0.2) (layer "F.Cu") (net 32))
 (segment (start 161.349999 143.350001) (end 159.95 144.75) (width 0.2) (layer "F.Cu") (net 7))
 (segment (start 153.65 142.45) (end 148.55 142.45) (width 0.2) (layer "F.Cu") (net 7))
 (segment (start 161.349999 141.65) (end 161.349999 143.350001) (width 0.2) (layer "F.Cu") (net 7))
 (segment (start 159.95 144.75) (end 155.95 144.75) (width 0.2) (layer "F.Cu") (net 7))
 (segment (start 155.95 144.75) (end 153.65 142.45) (width 0.2) (layer "F.Cu") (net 7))
 (segment (start 153.75 141.95) (end 156.05 144.25) (width 0.2) (layer "F.Cu") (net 6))
 (segment (start 148.55 141.95) (end 153.75 141.95) (width 0.2) (layer "F.Cu") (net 6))
 (segment (start 160.950001 143.147057) (end 160.950001 141.65) (width 0.2) (layer "F.Cu") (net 6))
 (segment (start 159.847058 144.25) (end 160.950001 143.147057) (width 0.2) (layer "F.Cu") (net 6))
 (segment (start 156.05 144.25) (end 159.847058 144.25) (width 0.2) (layer "F.Cu") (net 6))
 (segment (start 160.95 135.749999) (end 160.950001 135.75) (width 0.2) (layer "F.Cu") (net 30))
 (segment (start 148.55 133.95) (end 154.15 133.95) (width 0.2) (layer "F.Cu") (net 30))
 (segment (start 160.95 133.95) (end 160.95 135.749999) (width 0.2) (layer "F.Cu") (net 30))
 (segment (start 155.25 132.85) (end 159.85 132.85) (width 0.2) (layer "F.Cu") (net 30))
 (segment (start 154.15 133.95) (end 155.25 132.85) (width 0.2) (layer "F.Cu") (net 30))
 (segment (start 159.85 132.85) (end 160.95 133.95) (width 0.2) (layer "F.Cu") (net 30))
 (segment (start 160.55 135.75) (end 160.55 134.15) (width 0.2) (layer "F.Cu") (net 31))
 (segment (start 154.25 134.45) (end 148.55 134.45) (width 0.2) (layer "F.Cu") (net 31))
 (segment (start 159.65 133.25) (end 155.45 133.25) (width 0.2) (layer "F.Cu") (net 31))
 (segment (start 160.55 134.15) (end 159.65 133.25) (width 0.2) (layer "F.Cu") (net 31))
 (segment (start 155.45 133.25) (end 154.25 134.45) (width 0.2) (layer "F.Cu") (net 31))
 (segment (start 154.384314 137.45) (end 154.634314 137.7) (width 0.2) (layer "F.Cu") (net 39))
 (segment (start 148.55 137.45) (end 154.384314 137.45) (width 0.2) (layer "F.Cu") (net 39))
 (segment (start 154.634314 137.7) (end 158.2 137.7) (width 0.2) (layer "F.Cu") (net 39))
 (segment (start 159.515686 143.45) (end 156.65 143.45) (width 0.2) (layer "F.Cu") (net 4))
 (segment (start 148.55 140.95) (end 154.15 140.95) (width 0.2) (layer "F.Cu") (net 4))
 (segment (start 160.15 141.65) (end 160.15 142.815686) (width 0.2) (layer "F.Cu") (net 4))
 (segment (start 160.15 142.815686) (end 159.515686 143.45) (width 0.2) (layer "F.Cu") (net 4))
 (segment (start 154.15 140.95) (end 156.65 143.45) (width 0.2) (layer "F.Cu") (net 4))
 (segment (start 154.15 138.899999) (end 154.099999 138.95) (width 0.2) (layer "F.Cu") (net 42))
 (segment (start 158.2 138.899999) (end 154.15 138.899999) (width 0.2) (layer "F.Cu") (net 42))
 (segment (start 154.099999 138.95) (end 148.55 138.95) (width 0.2) (layer "F.Cu") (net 42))
 (segment (start 148.55 144.95) (end 153.718628 144.95) (width 0.2) (layer "F.Cu") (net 14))
 (segment (start 165.65 140.5) (end 164.1 140.5) (width 0.2) (layer "F.Cu") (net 14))
 (segment (start 166.55 144.4) (end 166.55 141.4) (width 0.2) (layer "F.Cu") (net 14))
 (segment (start 164.6 146.35) (end 166.55 144.4) (width 0.2) (layer "F.Cu") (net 14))
 (segment (start 153.718628 144.95) (end 155.118628 146.35) (width 0.2) (layer "F.Cu") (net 14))
 (segment (start 155.118628 146.35) (end 164.6 146.35) (width 0.2) (layer "F.Cu") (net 14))
 (segment (start 166.55 141.4) (end 165.65 140.5) (width 0.2) (layer "F.Cu") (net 14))
 (segment (start 154.65 131.65) (end 160.45 131.65) (width 0.2) (layer "F.Cu") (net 27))
 (segment (start 153.85 132.45) (end 154.65 131.65) (width 0.2) (layer "F.Cu") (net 27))
 (segment (start 148.55 132.45) (end 153.85 132.45) (width 0.2) (layer "F.Cu") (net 27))
 (segment (start 160.45 131.65) (end 162.15 133.35) (width 0.2) (layer "F.Cu") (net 27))
 (segment (start 162.15 133.35) (end 162.15 135.75) (width 0.2) (layer "F.Cu") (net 27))
 (segment (start 161.75 141.65) (end 161.75 143.55) (width 0.2) (layer "F.Cu") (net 8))
 (segment (start 153.45 142.95) (end 148.55 142.95) (width 0.2) (layer "F.Cu") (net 8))
 (segment (start 160.15 145.15) (end 155.65 145.15) (width 0.2) (layer "F.Cu") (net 8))
 (segment (start 155.65 145.15) (end 153.45 142.95) (width 0.2) (layer "F.Cu") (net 8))
 (segment (start 161.75 143.55) (end 160.15 145.15) (width 0.2) (layer "F.Cu") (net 8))
 (segment (start 167.35 141.068628) (end 165.981372 139.7) (width 0.2) (layer "F.Cu") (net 16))
 (segment (start 165.981372 139.7) (end 164.1 139.7) (width 0.2) (layer "F.Cu") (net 16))
 (segment (start 164.931372 147.15) (end 167.35 144.731372) (width 0.2) (layer "F.Cu") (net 16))
 (segment (start 167.35 144.731372) (end 167.35 141.068628) (width 0.2) (layer "F.Cu") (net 16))
 (segment (start 153.587256 145.95) (end 154.787256 147.15) (width 0.2) (layer "F.Cu") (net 16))
 (segment (start 154.787256 147.15) (end 164.931372 147.15) (width 0.2) (layer "F.Cu") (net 16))
 (segment (start 148.55 145.95) (end 153.587256 145.95) (width 0.2) (layer "F.Cu") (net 16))
 (segment (start 160.25 132.05) (end 154.85 132.05) (width 0.2) (layer "F.Cu") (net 28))
 (segment (start 161.75 133.55) (end 160.25 132.05) (width 0.2) (layer "F.Cu") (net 28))
 (segment (start 161.75 135.75) (end 161.75 133.55) (width 0.2) (layer "F.Cu") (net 28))
 (segment (start 153.95 132.95) (end 148.55 132.95) (width 0.2) (layer "F.Cu") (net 28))
 (segment (start 154.85 132.05) (end 153.95 132.95) (width 0.2) (layer "F.Cu") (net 28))
 (segment (start 159.681372 143.85) (end 160.55 142.981372) (width 0.2) (layer "F.Cu") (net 5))
 (segment (start 160.55 142.981372) (end 160.55 141.65) (width 0.2) (layer "F.Cu") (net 5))
 (segment (start 156.35 143.85) (end 159.681372 143.85) (width 0.2) (layer "F.Cu") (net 5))
 (segment (start 153.95 141.45) (end 156.35 143.85) (width 0.2) (layer "F.Cu") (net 5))
 (segment (start 148.55 141.45) (end 153.95 141.45) (width 0.2) (layer "F.Cu") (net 5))
 (segment (start 154.75 136.45) (end 155.2 136.9) (width 0.2) (layer "F.Cu") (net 37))
 (segment (start 148.55 136.45) (end 154.75 136.45) (width 0.2) (layer "F.Cu") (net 37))
 (segment (start 155.2 136.9) (end 158.2 136.9) (width 0.2) (layer "F.Cu") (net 37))
 (segment (start 166.95 141.234314) (end 165.815685 140.099999) (width 0.2) (layer "F.Cu") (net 15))
 (segment (start 165.815685 140.099999) (end 164.1 140.099999) (width 0.2) (layer "F.Cu") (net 15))
 (segment (start 153.652942 145.45) (end 154.952942 146.75) (width 0.2) (layer "F.Cu") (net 15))
 (segment (start 148.55 145.45) (end 153.652942 145.45) (width 0.2) (layer "F.Cu") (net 15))
 (segment (start 164.765686 146.75) (end 166.95 144.565686) (width 0.2) (layer "F.Cu") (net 15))
 (segment (start 154.952942 146.75) (end 164.765686 146.75) (width 0.2) (layer "F.Cu") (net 15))
 (segment (start 166.95 144.565686) (end 166.95 141.234314) (width 0.2) (layer "F.Cu") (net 15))
 (segment (start 154.55 135.45) (end 155.95 134.05) (width 0.2) (layer "F.Cu") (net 33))
 (segment (start 159.25 134.05) (end 159.750001 134.550001) (width 0.2) (layer "F.Cu") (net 33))
 (segment (start 159.750001 134.550001) (end 159.750001 135.75) (width 0.2) (layer "F.Cu") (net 33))
 (segment (start 148.55 135.45) (end 154.55 135.45) (width 0.2) (layer "F.Cu") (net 33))
 (segment (start 155.95 134.05) (end 159.25 134.05) (width 0.2) (layer "F.Cu") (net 33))
 (segment (start 148.55 136.95) (end 154.45 136.95) (width 0.2) (layer "F.Cu") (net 38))
 (segment (start 154.800001 137.300001) (end 158.2 137.300001) (width 0.2) (layer "F.Cu") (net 38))
 (segment (start 154.45 136.95) (end 154.800001 137.300001) (width 0.2) (layer "F.Cu") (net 38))
 (segment (start 165.097058 147.55) (end 167.75 144.897058) (width 0.2) (layer "F.Cu") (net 17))
 (segment (start 166.147058 139.3) (end 164.1 139.3) (width 0.2) (layer "F.Cu") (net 17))
 (segment (start 167.75 144.897058) (end 167.75 140.902942) (width 0.2) (layer "F.Cu") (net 17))
 (segment (start 153.52157 146.45) (end 154.62157 147.55) (width 0.2) (layer "F.Cu") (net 17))
 (segment (start 148.55 146.45) (end 153.52157 146.45) (width 0.2) (layer "F.Cu") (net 17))
 (segment (start 154.62157 147.55) (end 165.097058 147.55) (width 0.2) (layer "F.Cu") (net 17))
 (segment (start 167.75 140.902942) (end 166.147058 139.3) (width 0.2) (layer "F.Cu") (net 17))
 (segment (start 159.750001 142.649999) (end 159.750001 141.65) (width 0.2) (layer "F.Cu") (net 3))
 (segment (start 154.35 140.45) (end 156.95 143.05) (width 0.2) (layer "F.Cu") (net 3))
 (segment (start 156.95 143.05) (end 159.35 143.05) (width 0.2) (layer "F.Cu") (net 3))
 (segment (start 148.55 140.45) (end 154.35 140.45) (width 0.2) (layer "F.Cu") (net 3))
 (segment (start 159.35 143.05) (end 159.750001 142.649999) (width 0.2) (layer "F.Cu") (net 3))
 (segment (start 154.05 133.45) (end 148.55 133.45) (width 0.2) (layer "F.Cu") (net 29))
 (segment (start 155.05 132.45) (end 154.05 133.45) (width 0.2) (layer "F.Cu") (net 29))
 (segment (start 161.349999 133.784313) (end 160.015686 132.45) (width 0.2) (layer "F.Cu") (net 29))
 (segment (start 160.015686 132.45) (end 155.05 132.45) (width 0.2) (layer "F.Cu") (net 29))
 (segment (start 161.349999 135.75) (end 161.349999 133.784313) (width 0.2) (layer "F.Cu") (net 29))
 (segment (start 165.262744 147.95) (end 168.15 145.062744) (width 0.2) (layer "F.Cu") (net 18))
 (segment (start 154.455884 147.95) (end 165.262744 147.95) (width 0.2) (layer "F.Cu") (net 18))
 (segment (start 168.15 140.737256) (end 166.312745 138.900001) (width 0.2) (layer "F.Cu") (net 18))
 (segment (start 168.15 145.062744) (end 168.15 140.737256) (width 0.2) (layer "F.Cu") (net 18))
 (segment (start 153.455884 146.95) (end 154.455884 147.95) (width 0.2) (layer "F.Cu") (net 18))
 (segment (start 148.55 146.95) (end 153.455884 146.95) (width 0.2) (layer "F.Cu") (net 18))
 (segment (start 166.312745 138.900001) (end 164.1 138.900001) (width 0.2) (layer "F.Cu") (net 18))
 (segment (start 158.2 139.7) (end 154.5 139.7) (width 0.2) (layer "F.Cu") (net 44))
 (segment (start 154.25 139.95) (end 148.55 139.95) (width 0.2) (layer "F.Cu") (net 44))
 (segment (start 154.5 139.7) (end 154.25 139.95) (width 0.2) (layer "F.Cu") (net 44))
 (segment (start 158.2 139.3) (end 154.3 139.3) (width 0.2) (layer "F.Cu") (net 43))
 (segment (start 154.15 139.45) (end 148.55 139.45) (width 0.2) (layer "F.Cu") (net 43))
 (segment (start 154.3 139.3) (end 154.15 139.45) (width 0.2) (layer "F.Cu") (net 43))
 (segment (start 158.2 138.1) (end 154.4 138.1) (width 0.2) (layer "F.Cu") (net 40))
 (segment (start 154.25 137.95) (end 148.55 137.95) (width 0.2) (layer "F.Cu") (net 40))
 (segment (start 154.4 138.1) (end 154.25 137.95) (width 0.2) (layer "F.Cu") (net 40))
 (segment (start 155.284314 145.95) (end 153.284314 143.95) (width 0.2) (layer "F.Cu") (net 10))
 (segment (start 160.515686 145.95) (end 155.284314 145.95) (width 0.2) (layer "F.Cu") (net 10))
 (segment (start 162.549999 141.65) (end 162.549999 143.915687) (width 0.2) (layer "F.Cu") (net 10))
 (segment (start 153.284314 143.95) (end 148.55 143.95) (width 0.2) (layer "F.Cu") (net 10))
 (segment (start 162.549999 143.915687) (end 160.515686 145.95) (width 0.2) (layer "F.Cu") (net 10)))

